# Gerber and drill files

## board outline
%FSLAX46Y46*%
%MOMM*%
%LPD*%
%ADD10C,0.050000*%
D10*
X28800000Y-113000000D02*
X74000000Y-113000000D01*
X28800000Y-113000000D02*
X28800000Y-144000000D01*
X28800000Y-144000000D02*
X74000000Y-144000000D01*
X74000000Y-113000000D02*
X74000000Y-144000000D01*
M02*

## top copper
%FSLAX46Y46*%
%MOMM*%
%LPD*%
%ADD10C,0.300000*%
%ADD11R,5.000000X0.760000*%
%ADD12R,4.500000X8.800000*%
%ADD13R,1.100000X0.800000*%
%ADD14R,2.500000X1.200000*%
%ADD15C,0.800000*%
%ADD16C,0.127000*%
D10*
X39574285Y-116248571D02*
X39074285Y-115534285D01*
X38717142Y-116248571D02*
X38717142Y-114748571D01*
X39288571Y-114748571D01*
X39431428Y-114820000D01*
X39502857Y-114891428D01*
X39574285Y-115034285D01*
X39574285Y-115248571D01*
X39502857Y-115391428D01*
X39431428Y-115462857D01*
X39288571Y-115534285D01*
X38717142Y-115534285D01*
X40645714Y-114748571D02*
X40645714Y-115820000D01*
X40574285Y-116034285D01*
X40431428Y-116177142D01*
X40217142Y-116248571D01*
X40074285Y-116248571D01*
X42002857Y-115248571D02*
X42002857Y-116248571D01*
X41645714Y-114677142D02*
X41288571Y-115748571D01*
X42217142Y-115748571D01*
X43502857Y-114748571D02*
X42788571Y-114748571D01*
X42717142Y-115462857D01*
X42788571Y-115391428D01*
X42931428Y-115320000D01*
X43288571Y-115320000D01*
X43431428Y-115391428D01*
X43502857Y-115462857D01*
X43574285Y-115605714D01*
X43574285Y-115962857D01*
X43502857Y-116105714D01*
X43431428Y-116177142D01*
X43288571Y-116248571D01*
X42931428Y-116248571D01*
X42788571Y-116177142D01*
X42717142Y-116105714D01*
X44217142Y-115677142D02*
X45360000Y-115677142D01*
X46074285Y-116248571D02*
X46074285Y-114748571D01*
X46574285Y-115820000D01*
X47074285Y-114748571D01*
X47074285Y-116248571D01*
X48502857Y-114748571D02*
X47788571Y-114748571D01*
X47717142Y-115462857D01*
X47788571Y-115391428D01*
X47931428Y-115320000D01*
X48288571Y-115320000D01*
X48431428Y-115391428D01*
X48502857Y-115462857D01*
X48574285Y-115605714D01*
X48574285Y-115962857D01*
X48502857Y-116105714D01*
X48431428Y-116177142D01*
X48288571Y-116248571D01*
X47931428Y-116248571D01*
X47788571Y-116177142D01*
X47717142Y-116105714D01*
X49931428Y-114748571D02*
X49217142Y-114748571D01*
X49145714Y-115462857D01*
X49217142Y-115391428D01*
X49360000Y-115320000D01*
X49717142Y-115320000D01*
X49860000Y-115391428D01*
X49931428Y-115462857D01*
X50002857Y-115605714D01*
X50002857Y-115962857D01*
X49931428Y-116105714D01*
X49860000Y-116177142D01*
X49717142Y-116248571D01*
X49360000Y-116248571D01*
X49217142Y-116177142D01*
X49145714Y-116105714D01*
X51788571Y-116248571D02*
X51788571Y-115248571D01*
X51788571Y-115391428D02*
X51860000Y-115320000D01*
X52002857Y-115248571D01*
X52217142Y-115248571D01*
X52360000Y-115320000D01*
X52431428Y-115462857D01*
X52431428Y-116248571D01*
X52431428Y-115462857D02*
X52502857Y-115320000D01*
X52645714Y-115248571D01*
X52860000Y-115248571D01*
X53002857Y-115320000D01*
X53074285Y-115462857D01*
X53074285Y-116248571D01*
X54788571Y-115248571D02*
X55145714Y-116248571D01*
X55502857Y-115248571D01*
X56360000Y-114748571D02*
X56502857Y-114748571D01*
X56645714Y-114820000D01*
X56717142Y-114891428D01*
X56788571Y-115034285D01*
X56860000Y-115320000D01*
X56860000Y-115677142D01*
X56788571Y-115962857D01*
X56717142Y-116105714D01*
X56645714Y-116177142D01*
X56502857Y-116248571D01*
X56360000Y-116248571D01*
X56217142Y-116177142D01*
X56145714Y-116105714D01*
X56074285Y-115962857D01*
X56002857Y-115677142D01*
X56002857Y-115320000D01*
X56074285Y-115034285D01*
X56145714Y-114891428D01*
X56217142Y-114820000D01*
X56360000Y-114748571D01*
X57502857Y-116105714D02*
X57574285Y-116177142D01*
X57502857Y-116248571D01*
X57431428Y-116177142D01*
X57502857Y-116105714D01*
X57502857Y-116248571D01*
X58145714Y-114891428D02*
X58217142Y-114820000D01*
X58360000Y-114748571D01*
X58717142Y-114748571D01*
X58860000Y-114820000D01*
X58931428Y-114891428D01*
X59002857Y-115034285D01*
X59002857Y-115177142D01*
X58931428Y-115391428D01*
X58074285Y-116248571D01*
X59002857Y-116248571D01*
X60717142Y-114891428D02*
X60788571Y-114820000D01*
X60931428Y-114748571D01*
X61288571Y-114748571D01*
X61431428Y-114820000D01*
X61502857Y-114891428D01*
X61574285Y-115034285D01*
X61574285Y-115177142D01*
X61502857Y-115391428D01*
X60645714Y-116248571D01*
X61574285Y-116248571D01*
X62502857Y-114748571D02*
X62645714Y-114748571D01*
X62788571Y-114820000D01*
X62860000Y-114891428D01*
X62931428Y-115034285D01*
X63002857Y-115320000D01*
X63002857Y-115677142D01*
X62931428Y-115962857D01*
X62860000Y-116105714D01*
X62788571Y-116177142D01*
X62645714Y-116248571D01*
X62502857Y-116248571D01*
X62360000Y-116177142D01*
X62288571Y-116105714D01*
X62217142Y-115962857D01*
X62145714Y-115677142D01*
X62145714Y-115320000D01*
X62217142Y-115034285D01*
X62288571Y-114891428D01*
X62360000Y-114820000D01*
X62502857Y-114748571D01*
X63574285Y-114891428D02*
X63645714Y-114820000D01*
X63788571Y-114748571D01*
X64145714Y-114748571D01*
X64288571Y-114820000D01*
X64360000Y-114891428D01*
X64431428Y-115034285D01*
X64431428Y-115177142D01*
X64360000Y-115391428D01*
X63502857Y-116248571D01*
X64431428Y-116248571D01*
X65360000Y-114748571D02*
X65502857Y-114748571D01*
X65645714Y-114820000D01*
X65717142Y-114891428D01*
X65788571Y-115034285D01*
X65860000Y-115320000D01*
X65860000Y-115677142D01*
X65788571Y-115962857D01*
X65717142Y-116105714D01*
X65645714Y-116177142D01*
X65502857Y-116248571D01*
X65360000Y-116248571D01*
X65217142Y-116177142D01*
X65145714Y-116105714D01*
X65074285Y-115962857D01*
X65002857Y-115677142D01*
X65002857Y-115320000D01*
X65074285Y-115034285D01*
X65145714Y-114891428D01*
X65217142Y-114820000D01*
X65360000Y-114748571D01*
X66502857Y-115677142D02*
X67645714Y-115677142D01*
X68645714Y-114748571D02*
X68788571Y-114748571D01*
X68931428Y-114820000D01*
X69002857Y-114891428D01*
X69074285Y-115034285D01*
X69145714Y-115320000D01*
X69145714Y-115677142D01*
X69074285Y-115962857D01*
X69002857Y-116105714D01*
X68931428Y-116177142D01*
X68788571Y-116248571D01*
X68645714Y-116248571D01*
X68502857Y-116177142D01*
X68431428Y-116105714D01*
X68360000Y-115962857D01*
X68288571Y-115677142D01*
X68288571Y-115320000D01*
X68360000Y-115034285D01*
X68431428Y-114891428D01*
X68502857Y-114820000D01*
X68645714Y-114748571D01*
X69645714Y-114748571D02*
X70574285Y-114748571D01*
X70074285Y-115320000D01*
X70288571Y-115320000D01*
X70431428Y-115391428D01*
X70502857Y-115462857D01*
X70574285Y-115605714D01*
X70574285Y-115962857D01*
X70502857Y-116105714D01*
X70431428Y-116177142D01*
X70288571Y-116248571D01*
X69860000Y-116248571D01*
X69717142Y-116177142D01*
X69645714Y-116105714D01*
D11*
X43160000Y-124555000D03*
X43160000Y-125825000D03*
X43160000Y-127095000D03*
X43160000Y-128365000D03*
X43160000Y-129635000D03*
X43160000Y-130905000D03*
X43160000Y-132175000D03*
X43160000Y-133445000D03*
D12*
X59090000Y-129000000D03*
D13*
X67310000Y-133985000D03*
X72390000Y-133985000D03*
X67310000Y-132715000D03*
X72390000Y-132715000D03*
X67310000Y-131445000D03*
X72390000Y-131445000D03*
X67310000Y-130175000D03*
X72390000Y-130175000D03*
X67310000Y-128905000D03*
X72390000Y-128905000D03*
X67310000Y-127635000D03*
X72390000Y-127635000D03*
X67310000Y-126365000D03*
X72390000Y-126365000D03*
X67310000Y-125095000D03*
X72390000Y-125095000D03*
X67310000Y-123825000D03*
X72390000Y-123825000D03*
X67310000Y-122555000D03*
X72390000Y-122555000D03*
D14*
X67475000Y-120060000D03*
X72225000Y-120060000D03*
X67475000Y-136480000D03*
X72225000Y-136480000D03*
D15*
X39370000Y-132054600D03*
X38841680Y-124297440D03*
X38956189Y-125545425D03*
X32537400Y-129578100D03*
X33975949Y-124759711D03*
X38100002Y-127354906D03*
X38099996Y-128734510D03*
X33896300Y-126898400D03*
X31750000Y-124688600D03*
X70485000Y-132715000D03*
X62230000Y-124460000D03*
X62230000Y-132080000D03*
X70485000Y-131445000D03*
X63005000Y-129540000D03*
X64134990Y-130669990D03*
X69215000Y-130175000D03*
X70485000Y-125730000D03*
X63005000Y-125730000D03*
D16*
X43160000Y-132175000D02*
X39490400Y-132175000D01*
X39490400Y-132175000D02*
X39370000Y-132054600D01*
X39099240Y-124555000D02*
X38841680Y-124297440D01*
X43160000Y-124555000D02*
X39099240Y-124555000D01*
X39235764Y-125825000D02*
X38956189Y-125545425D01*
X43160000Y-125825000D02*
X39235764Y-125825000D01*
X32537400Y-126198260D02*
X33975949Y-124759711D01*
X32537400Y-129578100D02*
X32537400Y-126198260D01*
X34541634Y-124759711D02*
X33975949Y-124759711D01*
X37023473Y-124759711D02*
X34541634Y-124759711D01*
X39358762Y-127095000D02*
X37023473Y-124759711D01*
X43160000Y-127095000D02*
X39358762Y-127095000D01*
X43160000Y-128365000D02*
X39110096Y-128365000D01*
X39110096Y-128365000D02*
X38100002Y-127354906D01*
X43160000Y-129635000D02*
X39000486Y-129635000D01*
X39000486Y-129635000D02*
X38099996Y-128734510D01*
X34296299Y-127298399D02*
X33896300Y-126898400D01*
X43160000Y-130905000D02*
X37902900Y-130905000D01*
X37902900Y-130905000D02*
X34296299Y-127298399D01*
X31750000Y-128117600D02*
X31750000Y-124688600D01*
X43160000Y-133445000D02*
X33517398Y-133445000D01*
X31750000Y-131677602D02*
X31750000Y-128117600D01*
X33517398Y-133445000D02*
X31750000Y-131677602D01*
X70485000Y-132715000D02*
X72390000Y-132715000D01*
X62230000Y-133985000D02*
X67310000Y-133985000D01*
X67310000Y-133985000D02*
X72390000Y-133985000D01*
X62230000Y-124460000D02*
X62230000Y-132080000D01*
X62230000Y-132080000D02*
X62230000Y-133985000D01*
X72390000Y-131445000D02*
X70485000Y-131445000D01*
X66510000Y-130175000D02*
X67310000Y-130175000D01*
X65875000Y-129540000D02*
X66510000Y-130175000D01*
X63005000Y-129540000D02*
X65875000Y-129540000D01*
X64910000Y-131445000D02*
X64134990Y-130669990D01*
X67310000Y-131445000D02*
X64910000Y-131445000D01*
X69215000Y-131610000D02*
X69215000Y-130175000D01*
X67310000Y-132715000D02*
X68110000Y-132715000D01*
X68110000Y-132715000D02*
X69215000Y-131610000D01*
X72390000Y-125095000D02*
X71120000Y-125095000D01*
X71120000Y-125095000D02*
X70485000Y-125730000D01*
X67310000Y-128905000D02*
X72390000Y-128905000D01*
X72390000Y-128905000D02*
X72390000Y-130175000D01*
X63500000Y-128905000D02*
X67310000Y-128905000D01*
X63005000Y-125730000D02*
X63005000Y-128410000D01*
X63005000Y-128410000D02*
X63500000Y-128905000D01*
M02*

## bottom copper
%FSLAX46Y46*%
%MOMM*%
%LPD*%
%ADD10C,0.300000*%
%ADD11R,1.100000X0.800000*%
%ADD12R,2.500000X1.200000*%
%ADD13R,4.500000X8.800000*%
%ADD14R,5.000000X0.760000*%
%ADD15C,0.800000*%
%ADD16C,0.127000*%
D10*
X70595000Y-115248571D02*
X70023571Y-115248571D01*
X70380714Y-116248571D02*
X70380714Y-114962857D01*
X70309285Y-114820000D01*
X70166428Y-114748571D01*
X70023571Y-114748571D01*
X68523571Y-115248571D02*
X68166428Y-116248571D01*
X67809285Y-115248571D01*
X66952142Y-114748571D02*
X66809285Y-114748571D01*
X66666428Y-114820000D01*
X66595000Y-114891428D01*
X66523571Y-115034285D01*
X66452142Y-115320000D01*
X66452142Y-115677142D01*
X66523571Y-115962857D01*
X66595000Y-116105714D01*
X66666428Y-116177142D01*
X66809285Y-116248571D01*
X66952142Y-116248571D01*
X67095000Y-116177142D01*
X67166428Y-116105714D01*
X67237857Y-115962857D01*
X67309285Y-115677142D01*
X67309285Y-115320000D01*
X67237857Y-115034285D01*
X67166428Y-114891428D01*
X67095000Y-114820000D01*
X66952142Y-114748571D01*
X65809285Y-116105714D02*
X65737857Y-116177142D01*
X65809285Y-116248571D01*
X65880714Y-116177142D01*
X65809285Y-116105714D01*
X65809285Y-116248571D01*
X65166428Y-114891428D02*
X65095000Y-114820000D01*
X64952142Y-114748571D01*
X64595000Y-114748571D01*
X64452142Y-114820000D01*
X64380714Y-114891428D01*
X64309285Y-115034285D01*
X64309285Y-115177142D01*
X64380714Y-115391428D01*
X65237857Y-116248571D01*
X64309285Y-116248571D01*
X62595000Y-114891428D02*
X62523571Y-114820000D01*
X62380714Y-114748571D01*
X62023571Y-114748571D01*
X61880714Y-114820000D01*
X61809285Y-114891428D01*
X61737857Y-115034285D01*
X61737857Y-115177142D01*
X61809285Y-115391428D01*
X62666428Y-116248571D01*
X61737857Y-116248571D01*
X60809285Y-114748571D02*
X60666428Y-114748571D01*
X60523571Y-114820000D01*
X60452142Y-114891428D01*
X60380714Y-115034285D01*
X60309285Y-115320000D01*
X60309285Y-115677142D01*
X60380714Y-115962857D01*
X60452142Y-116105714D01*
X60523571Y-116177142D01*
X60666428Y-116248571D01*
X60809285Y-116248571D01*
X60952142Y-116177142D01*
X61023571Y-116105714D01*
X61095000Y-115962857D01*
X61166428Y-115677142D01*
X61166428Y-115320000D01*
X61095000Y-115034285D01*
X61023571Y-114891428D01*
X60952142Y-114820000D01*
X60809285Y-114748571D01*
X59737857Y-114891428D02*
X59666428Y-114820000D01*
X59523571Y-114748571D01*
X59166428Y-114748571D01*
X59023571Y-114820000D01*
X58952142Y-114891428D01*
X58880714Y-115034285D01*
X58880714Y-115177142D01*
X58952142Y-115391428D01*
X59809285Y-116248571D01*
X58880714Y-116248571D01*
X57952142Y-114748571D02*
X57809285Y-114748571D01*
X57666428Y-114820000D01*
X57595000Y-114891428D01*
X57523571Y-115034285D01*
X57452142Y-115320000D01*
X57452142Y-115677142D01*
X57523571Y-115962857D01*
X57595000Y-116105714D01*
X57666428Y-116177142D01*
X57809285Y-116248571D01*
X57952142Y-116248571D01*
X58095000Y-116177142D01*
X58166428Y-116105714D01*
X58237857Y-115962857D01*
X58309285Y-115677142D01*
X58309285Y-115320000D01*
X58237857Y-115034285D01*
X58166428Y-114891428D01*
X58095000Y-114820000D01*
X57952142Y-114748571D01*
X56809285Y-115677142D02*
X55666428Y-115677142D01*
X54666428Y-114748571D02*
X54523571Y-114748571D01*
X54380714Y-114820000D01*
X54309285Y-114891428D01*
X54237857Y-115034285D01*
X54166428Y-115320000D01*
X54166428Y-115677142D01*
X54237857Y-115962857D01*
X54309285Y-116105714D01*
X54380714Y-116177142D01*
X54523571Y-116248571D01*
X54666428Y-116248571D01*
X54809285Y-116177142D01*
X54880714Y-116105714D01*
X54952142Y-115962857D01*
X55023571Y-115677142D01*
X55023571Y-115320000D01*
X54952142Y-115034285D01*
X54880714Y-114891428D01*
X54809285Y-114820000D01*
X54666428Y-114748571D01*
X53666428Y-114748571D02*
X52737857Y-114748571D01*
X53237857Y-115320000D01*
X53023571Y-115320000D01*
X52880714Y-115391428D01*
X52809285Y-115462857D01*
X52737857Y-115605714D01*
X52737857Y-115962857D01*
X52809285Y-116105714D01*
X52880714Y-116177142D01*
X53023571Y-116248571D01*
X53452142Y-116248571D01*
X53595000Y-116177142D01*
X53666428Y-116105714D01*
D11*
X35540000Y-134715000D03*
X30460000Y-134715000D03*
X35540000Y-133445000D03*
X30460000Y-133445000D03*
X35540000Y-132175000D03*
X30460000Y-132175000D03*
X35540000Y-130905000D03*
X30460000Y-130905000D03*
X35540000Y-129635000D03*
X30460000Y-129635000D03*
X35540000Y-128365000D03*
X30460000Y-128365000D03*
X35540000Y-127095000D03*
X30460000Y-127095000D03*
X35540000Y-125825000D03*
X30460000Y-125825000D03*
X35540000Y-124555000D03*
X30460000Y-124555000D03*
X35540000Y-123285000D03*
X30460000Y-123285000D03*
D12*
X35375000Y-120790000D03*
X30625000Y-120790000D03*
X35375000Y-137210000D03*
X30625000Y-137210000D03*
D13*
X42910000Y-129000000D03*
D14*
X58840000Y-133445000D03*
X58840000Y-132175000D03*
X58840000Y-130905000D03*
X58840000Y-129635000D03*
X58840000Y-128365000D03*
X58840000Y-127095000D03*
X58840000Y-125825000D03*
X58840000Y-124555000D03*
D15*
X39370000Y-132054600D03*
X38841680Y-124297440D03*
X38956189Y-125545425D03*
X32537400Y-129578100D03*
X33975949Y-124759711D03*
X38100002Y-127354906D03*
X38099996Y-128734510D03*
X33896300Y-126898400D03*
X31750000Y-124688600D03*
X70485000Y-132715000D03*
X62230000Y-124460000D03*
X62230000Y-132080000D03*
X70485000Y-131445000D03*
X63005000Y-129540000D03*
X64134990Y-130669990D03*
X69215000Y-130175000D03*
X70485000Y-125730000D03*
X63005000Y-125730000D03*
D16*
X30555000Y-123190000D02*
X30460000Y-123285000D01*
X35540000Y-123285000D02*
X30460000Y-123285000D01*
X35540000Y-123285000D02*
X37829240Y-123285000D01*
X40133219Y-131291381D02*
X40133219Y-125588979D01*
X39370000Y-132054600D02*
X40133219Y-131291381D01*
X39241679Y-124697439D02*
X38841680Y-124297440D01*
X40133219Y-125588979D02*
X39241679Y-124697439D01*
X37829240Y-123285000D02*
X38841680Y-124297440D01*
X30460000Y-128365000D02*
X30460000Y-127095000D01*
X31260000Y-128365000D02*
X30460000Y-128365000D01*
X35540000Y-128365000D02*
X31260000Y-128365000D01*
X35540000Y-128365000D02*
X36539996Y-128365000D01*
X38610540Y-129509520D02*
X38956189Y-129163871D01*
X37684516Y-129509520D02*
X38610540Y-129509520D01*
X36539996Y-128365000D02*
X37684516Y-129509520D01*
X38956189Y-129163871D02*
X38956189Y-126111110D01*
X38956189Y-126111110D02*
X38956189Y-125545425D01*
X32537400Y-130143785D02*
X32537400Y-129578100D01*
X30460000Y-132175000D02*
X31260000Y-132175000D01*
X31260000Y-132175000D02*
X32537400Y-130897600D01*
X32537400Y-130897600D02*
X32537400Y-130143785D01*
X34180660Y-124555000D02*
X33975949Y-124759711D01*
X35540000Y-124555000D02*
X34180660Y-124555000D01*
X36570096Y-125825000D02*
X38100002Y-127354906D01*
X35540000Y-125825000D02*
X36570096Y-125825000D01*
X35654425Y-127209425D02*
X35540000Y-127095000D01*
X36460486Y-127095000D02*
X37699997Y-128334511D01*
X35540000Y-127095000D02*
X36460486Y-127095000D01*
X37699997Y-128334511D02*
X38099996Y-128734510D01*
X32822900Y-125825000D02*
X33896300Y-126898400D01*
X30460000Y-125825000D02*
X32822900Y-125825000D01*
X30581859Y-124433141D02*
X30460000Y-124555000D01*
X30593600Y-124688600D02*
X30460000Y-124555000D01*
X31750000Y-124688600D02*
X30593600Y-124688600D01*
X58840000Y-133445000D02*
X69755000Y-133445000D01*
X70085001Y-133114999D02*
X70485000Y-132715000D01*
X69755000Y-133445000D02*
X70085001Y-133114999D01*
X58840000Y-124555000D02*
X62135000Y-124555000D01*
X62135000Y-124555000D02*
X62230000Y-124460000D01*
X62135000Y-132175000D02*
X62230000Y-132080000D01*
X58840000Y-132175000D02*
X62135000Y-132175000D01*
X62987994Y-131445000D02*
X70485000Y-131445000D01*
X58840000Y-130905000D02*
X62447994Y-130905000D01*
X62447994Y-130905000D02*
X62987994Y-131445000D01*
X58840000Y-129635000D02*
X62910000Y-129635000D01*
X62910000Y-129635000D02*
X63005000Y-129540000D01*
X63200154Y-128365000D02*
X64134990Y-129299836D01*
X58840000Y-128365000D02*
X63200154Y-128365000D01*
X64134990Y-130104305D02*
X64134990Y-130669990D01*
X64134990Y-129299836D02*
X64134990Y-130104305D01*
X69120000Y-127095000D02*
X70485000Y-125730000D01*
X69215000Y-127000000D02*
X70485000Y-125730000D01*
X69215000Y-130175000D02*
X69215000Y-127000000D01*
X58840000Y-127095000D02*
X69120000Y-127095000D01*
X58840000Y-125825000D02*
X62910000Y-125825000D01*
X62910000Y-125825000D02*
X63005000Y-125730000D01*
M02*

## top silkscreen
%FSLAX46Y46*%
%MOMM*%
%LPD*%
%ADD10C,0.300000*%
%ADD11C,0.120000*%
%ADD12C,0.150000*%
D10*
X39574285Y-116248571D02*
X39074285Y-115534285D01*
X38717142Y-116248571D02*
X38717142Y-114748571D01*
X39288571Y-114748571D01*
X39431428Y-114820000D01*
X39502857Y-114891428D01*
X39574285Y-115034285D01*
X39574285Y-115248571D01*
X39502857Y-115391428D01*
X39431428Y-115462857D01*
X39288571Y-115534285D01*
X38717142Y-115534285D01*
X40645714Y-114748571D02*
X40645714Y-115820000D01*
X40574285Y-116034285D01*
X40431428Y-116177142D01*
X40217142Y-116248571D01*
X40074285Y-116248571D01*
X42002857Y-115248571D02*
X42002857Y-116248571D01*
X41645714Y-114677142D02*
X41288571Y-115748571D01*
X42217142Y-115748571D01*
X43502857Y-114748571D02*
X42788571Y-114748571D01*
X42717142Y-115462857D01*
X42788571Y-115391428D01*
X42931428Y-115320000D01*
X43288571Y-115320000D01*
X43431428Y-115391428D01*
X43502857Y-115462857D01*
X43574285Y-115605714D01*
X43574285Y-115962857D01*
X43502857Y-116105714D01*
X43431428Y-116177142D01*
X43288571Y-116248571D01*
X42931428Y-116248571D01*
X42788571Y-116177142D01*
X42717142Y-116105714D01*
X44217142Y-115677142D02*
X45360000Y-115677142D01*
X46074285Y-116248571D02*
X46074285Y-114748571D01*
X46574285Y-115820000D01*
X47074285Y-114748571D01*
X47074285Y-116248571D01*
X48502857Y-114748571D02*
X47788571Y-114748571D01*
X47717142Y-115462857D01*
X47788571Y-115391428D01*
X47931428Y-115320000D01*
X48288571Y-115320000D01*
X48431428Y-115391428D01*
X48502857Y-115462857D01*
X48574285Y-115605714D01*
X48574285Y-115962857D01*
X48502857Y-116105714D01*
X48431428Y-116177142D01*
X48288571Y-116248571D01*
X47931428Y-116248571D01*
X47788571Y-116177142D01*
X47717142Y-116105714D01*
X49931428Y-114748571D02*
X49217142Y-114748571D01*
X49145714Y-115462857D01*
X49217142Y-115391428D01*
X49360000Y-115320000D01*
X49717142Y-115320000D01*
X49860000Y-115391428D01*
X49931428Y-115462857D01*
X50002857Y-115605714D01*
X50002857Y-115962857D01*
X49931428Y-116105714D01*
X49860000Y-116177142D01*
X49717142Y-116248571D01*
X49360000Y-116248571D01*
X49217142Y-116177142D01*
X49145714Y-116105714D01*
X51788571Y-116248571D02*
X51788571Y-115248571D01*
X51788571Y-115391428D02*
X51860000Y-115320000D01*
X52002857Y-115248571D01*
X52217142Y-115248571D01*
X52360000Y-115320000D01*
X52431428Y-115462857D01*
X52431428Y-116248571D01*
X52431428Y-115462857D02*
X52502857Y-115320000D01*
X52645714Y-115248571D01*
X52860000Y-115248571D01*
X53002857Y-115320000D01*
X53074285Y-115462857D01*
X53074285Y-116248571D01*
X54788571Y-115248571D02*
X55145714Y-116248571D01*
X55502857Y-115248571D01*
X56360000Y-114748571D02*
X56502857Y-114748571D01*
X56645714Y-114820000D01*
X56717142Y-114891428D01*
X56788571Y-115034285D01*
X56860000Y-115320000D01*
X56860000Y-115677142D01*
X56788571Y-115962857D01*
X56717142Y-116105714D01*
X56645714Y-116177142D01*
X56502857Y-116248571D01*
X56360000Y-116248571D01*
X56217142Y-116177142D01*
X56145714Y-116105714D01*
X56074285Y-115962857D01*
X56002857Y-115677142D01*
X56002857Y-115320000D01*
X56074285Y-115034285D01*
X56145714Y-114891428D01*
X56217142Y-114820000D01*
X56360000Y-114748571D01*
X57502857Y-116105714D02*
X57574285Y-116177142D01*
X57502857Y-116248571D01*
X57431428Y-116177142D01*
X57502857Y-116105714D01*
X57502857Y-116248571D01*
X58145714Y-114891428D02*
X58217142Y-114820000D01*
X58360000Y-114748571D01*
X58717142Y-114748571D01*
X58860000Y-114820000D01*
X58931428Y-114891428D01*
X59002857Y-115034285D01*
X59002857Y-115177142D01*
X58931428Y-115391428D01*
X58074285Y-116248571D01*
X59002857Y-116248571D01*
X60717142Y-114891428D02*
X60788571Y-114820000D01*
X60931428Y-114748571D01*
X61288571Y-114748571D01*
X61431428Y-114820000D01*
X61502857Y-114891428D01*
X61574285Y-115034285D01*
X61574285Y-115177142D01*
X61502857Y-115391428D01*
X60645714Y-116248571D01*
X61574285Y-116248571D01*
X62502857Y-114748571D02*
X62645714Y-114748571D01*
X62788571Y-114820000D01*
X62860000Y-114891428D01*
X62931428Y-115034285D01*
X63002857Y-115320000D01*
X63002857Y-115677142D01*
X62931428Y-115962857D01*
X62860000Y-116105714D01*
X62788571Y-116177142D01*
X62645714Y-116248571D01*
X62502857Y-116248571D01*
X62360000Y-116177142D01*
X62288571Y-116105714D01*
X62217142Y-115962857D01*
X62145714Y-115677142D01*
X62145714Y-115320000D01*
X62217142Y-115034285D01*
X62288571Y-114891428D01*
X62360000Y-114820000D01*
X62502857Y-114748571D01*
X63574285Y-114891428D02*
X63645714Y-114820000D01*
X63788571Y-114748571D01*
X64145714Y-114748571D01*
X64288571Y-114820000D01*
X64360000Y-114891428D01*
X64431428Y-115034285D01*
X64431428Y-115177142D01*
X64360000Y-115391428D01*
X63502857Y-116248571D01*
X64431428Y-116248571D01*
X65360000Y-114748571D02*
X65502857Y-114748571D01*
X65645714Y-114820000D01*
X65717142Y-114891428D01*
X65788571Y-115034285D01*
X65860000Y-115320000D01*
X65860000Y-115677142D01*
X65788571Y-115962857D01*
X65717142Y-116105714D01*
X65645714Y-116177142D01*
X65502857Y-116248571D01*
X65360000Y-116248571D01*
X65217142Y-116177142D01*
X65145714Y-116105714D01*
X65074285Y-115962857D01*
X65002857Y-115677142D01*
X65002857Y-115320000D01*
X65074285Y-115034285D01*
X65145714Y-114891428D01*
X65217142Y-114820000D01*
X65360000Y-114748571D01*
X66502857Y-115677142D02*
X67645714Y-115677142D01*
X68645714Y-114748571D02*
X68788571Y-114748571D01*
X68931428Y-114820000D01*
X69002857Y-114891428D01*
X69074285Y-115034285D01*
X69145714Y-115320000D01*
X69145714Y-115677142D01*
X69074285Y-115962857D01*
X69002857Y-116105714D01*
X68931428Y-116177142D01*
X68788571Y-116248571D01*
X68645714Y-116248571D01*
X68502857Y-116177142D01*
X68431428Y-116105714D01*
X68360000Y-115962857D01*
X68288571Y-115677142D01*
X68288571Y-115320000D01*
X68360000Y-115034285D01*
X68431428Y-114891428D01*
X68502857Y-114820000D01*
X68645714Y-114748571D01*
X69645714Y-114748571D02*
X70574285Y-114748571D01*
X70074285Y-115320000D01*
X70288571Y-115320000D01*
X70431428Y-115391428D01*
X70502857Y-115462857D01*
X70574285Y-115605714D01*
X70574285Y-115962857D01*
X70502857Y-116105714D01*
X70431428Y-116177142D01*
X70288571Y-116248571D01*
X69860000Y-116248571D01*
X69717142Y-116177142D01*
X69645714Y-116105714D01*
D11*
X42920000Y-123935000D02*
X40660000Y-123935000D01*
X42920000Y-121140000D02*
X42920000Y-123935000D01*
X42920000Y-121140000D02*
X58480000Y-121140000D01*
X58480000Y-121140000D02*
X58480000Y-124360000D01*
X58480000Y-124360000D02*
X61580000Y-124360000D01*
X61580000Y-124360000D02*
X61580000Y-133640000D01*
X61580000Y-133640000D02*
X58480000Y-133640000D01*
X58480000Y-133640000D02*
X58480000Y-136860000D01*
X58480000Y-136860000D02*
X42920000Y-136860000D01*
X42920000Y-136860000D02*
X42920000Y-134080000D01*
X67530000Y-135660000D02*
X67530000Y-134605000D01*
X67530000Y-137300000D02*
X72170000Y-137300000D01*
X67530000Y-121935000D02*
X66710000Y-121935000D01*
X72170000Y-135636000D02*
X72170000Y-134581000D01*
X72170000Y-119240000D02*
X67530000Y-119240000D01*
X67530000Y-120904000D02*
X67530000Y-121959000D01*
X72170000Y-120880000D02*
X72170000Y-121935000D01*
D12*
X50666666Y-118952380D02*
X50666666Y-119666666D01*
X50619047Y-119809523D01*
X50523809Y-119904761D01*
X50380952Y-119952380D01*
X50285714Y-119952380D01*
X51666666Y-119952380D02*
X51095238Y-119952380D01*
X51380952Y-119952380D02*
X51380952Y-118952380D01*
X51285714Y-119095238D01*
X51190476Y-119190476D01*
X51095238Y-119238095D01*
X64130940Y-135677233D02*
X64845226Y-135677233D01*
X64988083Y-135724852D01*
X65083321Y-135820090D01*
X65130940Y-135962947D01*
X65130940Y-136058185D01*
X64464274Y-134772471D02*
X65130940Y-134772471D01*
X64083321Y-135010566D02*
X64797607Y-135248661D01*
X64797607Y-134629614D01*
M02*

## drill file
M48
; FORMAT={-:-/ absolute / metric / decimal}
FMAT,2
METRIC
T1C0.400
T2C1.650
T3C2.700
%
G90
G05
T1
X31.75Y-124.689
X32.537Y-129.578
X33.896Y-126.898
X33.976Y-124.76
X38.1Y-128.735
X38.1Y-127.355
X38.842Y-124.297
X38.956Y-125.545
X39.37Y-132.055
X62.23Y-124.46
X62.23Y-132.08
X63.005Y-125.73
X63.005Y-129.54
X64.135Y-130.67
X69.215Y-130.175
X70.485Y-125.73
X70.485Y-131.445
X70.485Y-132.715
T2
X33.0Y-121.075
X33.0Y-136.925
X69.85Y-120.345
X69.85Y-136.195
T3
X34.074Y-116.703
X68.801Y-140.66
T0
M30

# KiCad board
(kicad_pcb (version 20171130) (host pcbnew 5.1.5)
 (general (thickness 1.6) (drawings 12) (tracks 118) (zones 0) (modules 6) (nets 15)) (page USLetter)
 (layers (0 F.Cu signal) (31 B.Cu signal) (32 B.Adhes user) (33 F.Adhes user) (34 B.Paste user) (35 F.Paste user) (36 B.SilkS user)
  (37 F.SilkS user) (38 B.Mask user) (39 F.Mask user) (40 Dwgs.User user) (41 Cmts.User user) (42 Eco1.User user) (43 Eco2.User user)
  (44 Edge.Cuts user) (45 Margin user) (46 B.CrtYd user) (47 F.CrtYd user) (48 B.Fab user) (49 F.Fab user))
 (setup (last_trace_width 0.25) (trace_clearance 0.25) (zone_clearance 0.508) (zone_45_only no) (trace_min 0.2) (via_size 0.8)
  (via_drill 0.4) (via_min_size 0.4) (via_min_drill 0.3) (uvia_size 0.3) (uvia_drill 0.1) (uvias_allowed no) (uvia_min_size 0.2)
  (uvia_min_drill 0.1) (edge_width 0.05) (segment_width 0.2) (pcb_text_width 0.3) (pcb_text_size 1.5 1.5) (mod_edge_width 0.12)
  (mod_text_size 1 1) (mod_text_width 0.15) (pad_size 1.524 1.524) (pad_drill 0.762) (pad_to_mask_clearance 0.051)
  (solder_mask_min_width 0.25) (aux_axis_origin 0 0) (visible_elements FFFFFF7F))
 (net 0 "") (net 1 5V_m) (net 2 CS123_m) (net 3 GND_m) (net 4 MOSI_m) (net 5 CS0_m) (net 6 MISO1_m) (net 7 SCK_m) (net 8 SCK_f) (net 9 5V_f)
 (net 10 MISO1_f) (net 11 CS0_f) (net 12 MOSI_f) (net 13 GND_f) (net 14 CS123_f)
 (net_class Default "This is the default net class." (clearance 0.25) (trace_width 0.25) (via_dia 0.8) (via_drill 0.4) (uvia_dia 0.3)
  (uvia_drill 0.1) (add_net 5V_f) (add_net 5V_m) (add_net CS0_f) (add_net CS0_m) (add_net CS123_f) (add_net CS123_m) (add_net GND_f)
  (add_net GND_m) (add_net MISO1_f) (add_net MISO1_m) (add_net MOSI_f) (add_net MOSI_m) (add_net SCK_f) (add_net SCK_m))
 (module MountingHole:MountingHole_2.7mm (layer F.Cu) (at 68.80098 140.66012)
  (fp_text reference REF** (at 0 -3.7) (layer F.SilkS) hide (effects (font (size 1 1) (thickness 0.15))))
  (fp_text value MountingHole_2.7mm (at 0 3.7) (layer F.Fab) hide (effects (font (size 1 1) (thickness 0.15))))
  (pad 1 np_thru_hole circle (at 0 0) (size 2.7 2.7) (drill 2.7) (layers *.Cu *.Mask)))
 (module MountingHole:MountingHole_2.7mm (layer F.Cu) (at 34.0741 116.70284)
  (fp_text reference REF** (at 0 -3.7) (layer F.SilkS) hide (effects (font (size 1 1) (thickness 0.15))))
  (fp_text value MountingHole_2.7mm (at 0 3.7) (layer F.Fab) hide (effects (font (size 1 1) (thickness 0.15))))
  (pad 1 np_thru_hole circle (at 0 0) (size 2.7 2.7) (drill 2.7) (layers *.Cu *.Mask)))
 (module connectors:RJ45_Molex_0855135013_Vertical (layer F.Cu) (at 51 129)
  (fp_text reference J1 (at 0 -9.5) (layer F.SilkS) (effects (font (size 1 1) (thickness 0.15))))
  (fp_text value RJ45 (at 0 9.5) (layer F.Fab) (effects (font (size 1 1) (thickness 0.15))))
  (fp_line (start -8.08 -5.065) (end -10.34 -5.065) (layer F.SilkS) (width 0.12))
  (fp_line (start -8.08 -7.86) (end -8.08 -5.065) (layer F.SilkS) (width 0.12))
  (fp_line (start -8.08 -7.86) (end 7.48 -7.86) (layer F.SilkS) (width 0.12))
  (fp_line (start 7.48 -7.86) (end 7.48 -4.64) (layer F.SilkS) (width 0.12))
  (fp_line (start 7.48 -4.64) (end 10.58 -4.64) (layer F.SilkS) (width 0.12))
  (fp_line (start 10.58 -4.64) (end 10.58 4.64) (layer F.SilkS) (width 0.12))
  (fp_line (start 10.58 4.64) (end 7.48 4.64) (layer F.SilkS) (width 0.12))
  (fp_line (start 7.48 4.64) (end 7.48 7.86) (layer F.SilkS) (width 0.12))
  (fp_line (start 7.48 7.86) (end -8.08 7.86) (layer F.SilkS) (width 0.12))
  (fp_line (start -8.08 7.86) (end -8.08 5.08) (layer F.SilkS) (width 0.12))
  (pad 1 smd rect (at -7.84 -4.445 270) (size 0.76 5) (layers F.Cu F.Paste F.Mask) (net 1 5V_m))
  (pad 2 smd rect (at -7.84 -3.175 270) (size 0.76 5) (layers F.Cu F.Paste F.Mask) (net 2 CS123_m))
  (pad 3 smd rect (at -7.84 -1.905 270) (size 0.76 5) (layers F.Cu F.Paste F.Mask) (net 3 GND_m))
  (pad 4 smd rect (at -7.84 -0.635 270) (size 0.76 5) (layers F.Cu F.Paste F.Mask) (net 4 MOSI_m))
  (pad 5 smd rect (at -7.84 0.635 270) (size 0.76 5) (layers F.Cu F.Paste F.Mask) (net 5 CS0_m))
  (pad 6 smd rect (at -7.84 1.905 270) (size 0.76 5) (layers F.Cu F.Paste F.Mask) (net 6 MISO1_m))
  (pad 7 smd rect (at -7.84 3.175 270) (size 0.76 5) (layers F.Cu F.Paste F.Mask) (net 1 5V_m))
  (pad 8 smd rect (at -7.84 4.445 270) (size 0.76 5) (layers F.Cu F.Paste F.Mask) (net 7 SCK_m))
  (pad L smd rect (at 8.09 0 270) (size 8.8 4.5) (layers F.Cu F.Paste F.Mask)))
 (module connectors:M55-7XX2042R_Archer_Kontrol (layer B.Cu) (at 33 129 90)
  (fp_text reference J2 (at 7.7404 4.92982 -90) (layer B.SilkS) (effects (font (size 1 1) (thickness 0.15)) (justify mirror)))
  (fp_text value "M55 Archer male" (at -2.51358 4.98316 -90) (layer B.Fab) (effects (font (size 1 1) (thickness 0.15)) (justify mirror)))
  (pad 1 smd rect (at -5.715 2.54 90) (size 0.8 1.1) (layers B.Cu B.Paste B.Mask))
  (pad 2 smd rect (at -5.715 -2.54 90) (size 0.8 1.1) (layers B.Cu B.Paste B.Mask))
  (pad 3 smd rect (at -4.445 2.54 90) (size 0.8 1.1) (layers B.Cu B.Paste B.Mask))
  (pad 4 smd rect (at -4.445 -2.54 90) (size 0.8 1.1) (layers B.Cu B.Paste B.Mask))
  (pad 5 smd rect (at -3.175 2.54 90) (size 0.8 1.1) (layers B.Cu B.Paste B.Mask))
  (pad 6 smd rect (at -3.175 -2.54 90) (size 0.8 1.1) (layers B.Cu B.Paste B.Mask) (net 3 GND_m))
  (pad 7 smd rect (at -1.905 2.54 90) (size 0.8 1.1) (layers B.Cu B.Paste B.Mask))
  (pad 8 smd rect (at -1.905 -2.54 90) (size 0.8 1.1) (layers B.Cu B.Paste B.Mask))
  (pad 9 smd rect (at -0.635 2.54 90) (size 0.8 1.1) (layers B.Cu B.Paste B.Mask))
  (pad 10 smd rect (at -0.635 -2.54 90) (size 0.8 1.1) (layers B.Cu B.Paste B.Mask))
  (pad 11 smd rect (at 0.635 2.54 90) (size 0.8 1.1) (layers B.Cu B.Paste B.Mask) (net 2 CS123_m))
  (pad 12 smd rect (at 0.635 -2.54 90) (size 0.8 1.1) (layers B.Cu B.Paste B.Mask) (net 2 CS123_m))
  (pad 13 smd rect (at 1.905 2.54 90) (size 0.8 1.1) (layers B.Cu B.Paste B.Mask) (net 5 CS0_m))
  (pad 14 smd rect (at 1.905 -2.54 90) (size 0.8 1.1) (layers B.Cu B.Paste B.Mask) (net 2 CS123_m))
  (pad 15 smd rect (at 3.175 2.54 90) (size 0.8 1.1) (layers B.Cu B.Paste B.Mask) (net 4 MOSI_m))
  (pad 16 smd rect (at 3.175 -2.54 90) (size 0.8 1.1) (layers B.Cu B.Paste B.Mask) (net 6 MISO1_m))
  (pad 17 smd rect (at 4.445 2.54 90) (size 0.8 1.1) (layers B.Cu B.Paste B.Mask) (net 3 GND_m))
  (pad 18 smd rect (at 4.445 -2.54 90) (size 0.8 1.1) (layers B.Cu B.Paste B.Mask) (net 7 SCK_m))
  (pad 19 smd rect (at 5.715 2.54 90) (size 0.8 1.1) (layers B.Cu B.Paste B.Mask) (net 1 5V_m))
  (pad 20 smd rect (at 5.715 -2.54 90) (size 0.8 1.1) (layers B.Cu B.Paste B.Mask) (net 1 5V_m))
  (pad "" np_thru_hole circle (at 7.925 0 90) (size 1.65 1.65) (drill 1.65) (layers *.Cu *.Mask))
  (pad "" np_thru_hole circle (at -7.925 0 90) (size 1.65 1.65) (drill 1.65) (layers *.Cu *.Mask))
  (pad "" smd rect (at 8.21 2.375 90) (size 1.2 2.5) (layers B.Cu B.Paste B.Mask))
  (pad "" smd rect (at 8.21 -2.375 90) (size 1.2 2.5) (layers B.Cu B.Paste B.Mask))
  (pad "" smd rect (at -8.21 2.375 90) (size 1.2 2.5) (layers B.Cu B.Paste B.Mask))
  (pad "" smd rect (at -8.21 -2.375 90) (size 1.2 2.5) (layers B.Cu B.Paste B.Mask)))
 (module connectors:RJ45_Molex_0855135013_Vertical (layer B.Cu) (at 51 129 180)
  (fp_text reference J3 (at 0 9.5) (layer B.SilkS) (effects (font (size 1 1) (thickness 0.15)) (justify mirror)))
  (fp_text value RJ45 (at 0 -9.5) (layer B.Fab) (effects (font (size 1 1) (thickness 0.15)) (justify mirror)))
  (pad L smd rect (at 8.09 0 270) (size 8.8 4.5) (layers B.Cu B.Paste B.Mask))
  (pad 8 smd rect (at -7.84 -4.445 270) (size 0.76 5) (layers B.Cu B.Paste B.Mask) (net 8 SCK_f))
  (pad 7 smd rect (at -7.84 -3.175 270) (size 0.76 5) (layers B.Cu B.Paste B.Mask) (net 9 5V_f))
  (pad 6 smd rect (at -7.84 -1.905 270) (size 0.76 5) (layers B.Cu B.Paste B.Mask) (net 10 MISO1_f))
  (pad 5 smd rect (at -7.84 -0.635 270) (size 0.76 5) (layers B.Cu B.Paste B.Mask) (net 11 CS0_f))
  (pad 4 smd rect (at -7.84 0.635 270) (size 0.76 5) (layers B.Cu B.Paste B.Mask) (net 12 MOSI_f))
  (pad 3 smd rect (at -7.84 1.905 270) (size 0.76 5) (layers B.Cu B.Paste B.Mask) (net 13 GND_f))
  (pad 2 smd rect (at -7.84 3.175 270) (size 0.76 5) (layers B.Cu B.Paste B.Mask) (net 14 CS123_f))
  (pad 1 smd rect (at -7.84 4.445 270) (size 0.76 5) (layers B.Cu B.Paste B.Mask) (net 9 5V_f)))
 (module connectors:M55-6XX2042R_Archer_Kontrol (layer F.Cu) (at 69.85 128.27 90)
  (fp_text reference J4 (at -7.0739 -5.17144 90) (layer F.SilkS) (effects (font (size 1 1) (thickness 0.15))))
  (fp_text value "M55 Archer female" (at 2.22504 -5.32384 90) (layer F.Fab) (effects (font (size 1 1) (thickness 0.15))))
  (fp_line (start -7.39 -2.32) (end -6.335 -2.32) (layer F.SilkS) (width 0.12))
  (fp_line (start -9.03 -2.32) (end -9.03 2.32) (layer F.SilkS) (width 0.12))
  (fp_line (start 6.335 -2.32) (end 6.335 -3.14) (layer F.SilkS) (width 0.12))
  (fp_line (start -7.366 2.32) (end -6.311 2.32) (layer F.SilkS) (width 0.12))
  (fp_line (start 9.03 2.32) (end 9.03 -2.32) (layer F.SilkS) (width 0.12))
  (fp_line (start 7.366 -2.32) (end 6.311 -2.32) (layer F.SilkS) (width 0.12))
  (fp_line (start 7.39 2.32) (end 6.335 2.32) (layer F.SilkS) (width 0.12))
  (pad 19 smd rect (at -5.715 -2.54 90) (size 0.8 1.1) (layers F.Cu F.Paste F.Mask) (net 9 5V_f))
  (pad 20 smd rect (at -5.715 2.54 90) (size 0.8 1.1) (layers F.Cu F.Paste F.Mask) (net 9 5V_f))
  (pad 17 smd rect (at -4.445 -2.54 90) (size 0.8 1.1) (layers F.Cu F.Paste F.Mask) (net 13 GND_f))
  (pad 18 smd rect (at -4.445 2.54 90) (size 0.8 1.1) (layers F.Cu F.Paste F.Mask) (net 8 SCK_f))
  (pad 15 smd rect (at -3.175 -2.54 90) (size 0.8 1.1) (layers F.Cu F.Paste F.Mask) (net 12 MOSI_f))
  (pad 16 smd rect (at -3.175 2.54 90) (size 0.8 1.1) (layers F.Cu F.Paste F.Mask) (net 10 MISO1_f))
  (pad 13 smd rect (at -1.905 -2.54 90) (size 0.8 1.1) (layers F.Cu F.Paste F.Mask) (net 11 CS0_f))
  (pad 14 smd rect (at -1.905 2.54 90) (size 0.8 1.1) (layers F.Cu F.Paste F.Mask) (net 14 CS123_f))
  (pad 11 smd rect (at -0.635 -2.54 90) (size 0.8 1.1) (layers F.Cu F.Paste F.Mask) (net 14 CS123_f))
  (pad 12 smd rect (at -0.635 2.54 90) (size 0.8 1.1) (layers F.Cu F.Paste F.Mask) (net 14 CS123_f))
  (pad 9 smd rect (at 0.635 -2.54 90) (size 0.8 1.1) (layers F.Cu F.Paste F.Mask))
  (pad 10 smd rect (at 0.635 2.54 90) (size 0.8 1.1) (layers F.Cu F.Paste F.Mask))
  (pad 7 smd rect (at 1.905 -2.54 90) (size 0.8 1.1) (layers F.Cu F.Paste F.Mask))
  (pad 8 smd rect (at 1.905 2.54 90) (size 0.8 1.1) (layers F.Cu F.Paste F.Mask))
  (pad 5 smd rect (at 3.175 -2.54 90) (size 0.8 1.1) (layers F.Cu F.Paste F.Mask))
  (pad 6 smd rect (at 3.175 2.54 90) (size 0.8 1.1) (layers F.Cu F.Paste F.Mask) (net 13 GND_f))
  (pad 3 smd rect (at 4.445 -2.54 90) (size 0.8 1.1) (layers F.Cu F.Paste F.Mask))
  (pad 4 smd rect (at 4.445 2.54 90) (size 0.8 1.1) (layers F.Cu F.Paste F.Mask))
  (pad 1 smd rect (at 5.715 -2.54 90) (size 0.8 1.1) (layers F.Cu F.Paste F.Mask))
  (pad 2 smd rect (at 5.715 2.54 90) (size 0.8 1.1) (layers F.Cu F.Paste F.Mask))
  (pad "" np_thru_hole circle (at 7.925 0 90) (size 1.65 1.65) (drill 1.65) (layers *.Cu *.Mask))
  (pad "" np_thru_hole circle (at -7.925 0 90) (size 1.65 1.65) (drill 1.65) (layers *.Cu *.Mask))
  (pad "" smd rect (at 8.21 -2.375 90) (size 1.2 2.5) (layers F.Cu F.Paste F.Mask))
  (pad "" smd rect (at 8.21 2.375 90) (size 1.2 2.5) (layers F.Cu F.Paste F.Mask))
  (pad "" smd rect (at -8.21 -2.375 90) (size 1.2 2.5) (layers F.Cu F.Paste F.Mask))
  (pad "" smd rect (at -8.21 2.375 90) (size 1.2 2.5) (layers F.Cu F.Paste F.Mask)))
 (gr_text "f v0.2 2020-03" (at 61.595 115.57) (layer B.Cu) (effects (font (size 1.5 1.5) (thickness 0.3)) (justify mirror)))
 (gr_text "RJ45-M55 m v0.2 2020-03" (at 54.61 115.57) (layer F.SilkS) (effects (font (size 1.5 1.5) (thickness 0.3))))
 (gr_line (start 28.8 113) (end 74 113) (layer Edge.Cuts) (width 0.05))
 (gr_line (start 28.8 113) (end 28.8 144) (layer Edge.Cuts) (width 0.05))
 (gr_line (start 28.8 144) (end 74 144) (layer Edge.Cuts) (width 0.05))
 (gr_line (start 74 113) (end 74 144) (layer Edge.Cuts) (width 0.05))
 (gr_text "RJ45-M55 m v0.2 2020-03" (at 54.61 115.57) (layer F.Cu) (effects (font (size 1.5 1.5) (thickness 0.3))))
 (segment (start 30.555 123.19) (end 30.46 123.285) (width 0.127) (layer B.Cu) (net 1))
 (segment (start 35.54 123.285) (end 30.46 123.285) (width 0.127) (layer B.Cu) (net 1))
 (segment (start 43.16 132.175) (end 39.4904 132.175) (width 0.127) (layer F.Cu) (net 1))
 (segment (start 39.4904 132.175) (end 39.37 132.0546) (width 0.127) (layer F.Cu) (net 1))
 (via (at 39.37 132.0546) (size 0.8) (drill 0.4) (layers F.Cu B.Cu) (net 1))
 (segment (start 35.54 123.285) (end 37.82924 123.285) (width 0.127) (layer B.Cu) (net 1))
 (segment (start 39.09924 124.555) (end 38.84168 124.29744) (width 0.127) (layer F.Cu) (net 1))
 (segment (start 40.133219 131.291381) (end 40.133219 125.588979) (width 0.127) (layer B.Cu) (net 1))
 (segment (start 39.37 132.0546) (end 40.133219 131.291381) (width 0.127) (layer B.Cu) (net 1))
 (via (at 38.84168 124.29744) (size 0.8) (drill 0.4) (layers F.Cu B.Cu) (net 1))
 (segment (start 39.241679 124.697439) (end 38.84168 124.29744) (width 0.127) (layer B.Cu) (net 1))
 (segment (start 43.16 124.555) (end 39.09924 124.555) (width 0.127) (layer F.Cu) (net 1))
 (segment (start 40.133219 125.588979) (end 39.241679 124.697439) (width 0.127) (layer B.Cu) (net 1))
 (segment (start 37.82924 123.285) (end 38.84168 124.29744) (width 0.127) (layer B.Cu) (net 1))
 (segment (start 30.46 128.365) (end 30.46 127.095) (width 0.127) (layer B.Cu) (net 2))
 (segment (start 31.26 128.365) (end 30.46 128.365) (width 0.127) (layer B.Cu) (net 2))
 (segment (start 35.54 128.365) (end 31.26 128.365) (width 0.127) (layer B.Cu) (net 2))
 (segment (start 35.54 128.365) (end 36.539996 128.365) (width 0.127) (layer B.Cu) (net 2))
 (segment (start 39.235764 125.825) (end 38.956189 125.545425) (width 0.127) (layer F.Cu) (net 2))
 (segment (start 38.61054 129.50952) (end 38.956189 129.163871) (width 0.127) (layer B.Cu) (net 2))
 (segment (start 37.684516 129.50952) (end 38.61054 129.50952) (width 0.127) (layer B.Cu) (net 2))
 (via (at 38.956189 125.545425) (size 0.8) (drill 0.4) (layers F.Cu B.Cu) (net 2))
 (segment (start 43.16 125.825) (end 39.235764 125.825) (width 0.127) (layer F.Cu) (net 2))
 (segment (start 36.539996 128.365) (end 37.684516 129.50952) (width 0.127) (layer B.Cu) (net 2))
 (segment (start 38.956189 129.163871) (end 38.956189 126.11111) (width 0.127) (layer B.Cu) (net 2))
 (segment (start 38.956189 126.11111) (end 38.956189 125.545425) (width 0.127) (layer B.Cu) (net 2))
 (via (at 32.5374 129.5781) (size 0.8) (drill 0.4) (layers F.Cu B.Cu) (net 3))
 (segment (start 32.5374 130.143785) (end 32.5374 129.5781) (width 0.127) (layer B.Cu) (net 3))
 (segment (start 30.46 132.175) (end 31.26 132.175) (width 0.127) (layer B.Cu) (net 3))
 (segment (start 31.26 132.175) (end 32.5374 130.8976) (width 0.127) (layer B.Cu) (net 3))
 (segment (start 32.5374 130.8976) (end 32.5374 130.143785) (width 0.127) (layer B.Cu) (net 3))
 (segment (start 34.18066 124.555) (end 33.975949 124.759711) (width 0.127) (layer B.Cu) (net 3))
 (via (at 33.975949 124.759711) (size 0.8) (drill 0.4) (layers F.Cu B.Cu) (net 3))
 (segment (start 35.54 124.555) (end 34.18066 124.555) (width 0.127) (layer B.Cu) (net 3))
 (segment (start 32.5374 126.19826) (end 33.975949 124.759711) (width 0.127) (layer F.Cu) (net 3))
 (segment (start 32.5374 129.5781) (end 32.5374 126.19826) (width 0.127) (layer F.Cu) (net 3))
 (segment (start 34.541634 124.759711) (end 33.975949 124.759711) (width 0.127) (layer F.Cu) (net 3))
 (segment (start 37.023473 124.759711) (end 34.541634 124.759711) (width 0.127) (layer F.Cu) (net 3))
 (segment (start 39.358762 127.095) (end 37.023473 124.759711) (width 0.127) (layer F.Cu) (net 3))
 (segment (start 43.16 127.095) (end 39.358762 127.095) (width 0.127) (layer F.Cu) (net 3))
 (segment (start 43.16 128.365) (end 39.110096 128.365) (width 0.127) (layer F.Cu) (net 4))
 (segment (start 36.570096 125.825) (end 38.100002 127.354906) (width 0.127) (layer B.Cu) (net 4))
 (segment (start 35.54 125.825) (end 36.570096 125.825) (width 0.127) (layer B.Cu) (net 4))
 (segment (start 39.110096 128.365) (end 38.100002 127.354906) (width 0.127) (layer F.Cu) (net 4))
 (via (at 38.100002 127.354906) (size 0.8) (drill 0.4) (layers F.Cu B.Cu) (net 4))
 (segment (start 35.654425 127.209425) (end 35.54 127.095) (width 0.127) (layer B.Cu) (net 5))
 (via (at 38.099996 128.73451) (size 0.8) (drill 0.4) (layers F.Cu B.Cu) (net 5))
 (segment (start 36.460486 127.095) (end 37.699997 128.334511) (width 0.127) (layer B.Cu) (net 5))
 (segment (start 43.16 129.635) (end 39.000486 129.635) (width 0.127) (layer F.Cu) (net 5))
 (segment (start 35.54 127.095) (end 36.460486 127.095) (width 0.127) (layer B.Cu) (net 5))
 (segment (start 37.699997 128.334511) (end 38.099996 128.73451) (width 0.127) (layer B.Cu) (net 5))
 (segment (start 39.000486 129.635) (end 38.099996 128.73451) (width 0.127) (layer F.Cu) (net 5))
 (segment (start 34.296299 127.298399) (end 33.8963 126.8984) (width 0.127) (layer F.Cu) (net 6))
 (segment (start 43.16 130.905) (end 37.9029 130.905) (width 0.127) (layer F.Cu) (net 6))
 (segment (start 37.9029 130.905) (end 34.296299 127.298399) (width 0.127) (layer F.Cu) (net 6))
 (via (at 33.8963 126.8984) (size 0.8) (drill 0.4) (layers F.Cu B.Cu) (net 6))
 (segment (start 32.8229 125.825) (end 33.8963 126.8984) (width 0.127) (layer B.Cu) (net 6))
 (segment (start 30.46 125.825) (end 32.8229 125.825) (width 0.127) (layer B.Cu) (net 6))
 (segment (start 30.581859 124.433141) (end 30.46 124.555) (width 0.127) (layer B.Cu) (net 7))
 (via (at 31.75 124.6886) (size 0.8) (drill 0.4) (layers F.Cu B.Cu) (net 7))
 (segment (start 30.5936 124.6886) (end 30.46 124.555) (width 0.127) (layer B.Cu) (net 7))
 (segment (start 31.75 124.6886) (end 30.5936 124.6886) (width 0.127) (layer B.Cu) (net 7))
 (segment (start 31.75 128.1176) (end 31.75 124.6886) (width 0.127) (layer F.Cu) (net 7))
 (segment (start 43.16 133.445) (end 33.517398 133.445) (width 0.127) (layer F.Cu) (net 7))
 (segment (start 31.75 131.677602) (end 31.75 128.1176) (width 0.127) (layer F.Cu) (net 7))
 (segment (start 33.517398 133.445) (end 31.75 131.677602) (width 0.127) (layer F.Cu) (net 7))
 (via (at 70.485 132.715) (size 0.8) (drill 0.4) (layers F.Cu B.Cu) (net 8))
 (segment (start 70.485 132.715) (end 72.39 132.715) (width 0.127) (layer F.Cu) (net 8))
 (segment (start 58.84 133.445) (end 69.755 133.445) (width 0.127) (layer B.Cu) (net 8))
 (segment (start 70.085001 133.114999) (end 70.485 132.715) (width 0.127) (layer B.Cu) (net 8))
 (segment (start 69.755 133.445) (end 70.085001 133.114999) (width 0.127) (layer B.Cu) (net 8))
 (via (at 62.23 124.46) (size 0.8) (drill 0.4) (layers F.Cu B.Cu) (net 9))
 (segment (start 58.84 124.555) (end 62.135 124.555) (width 0.127) (layer B.Cu) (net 9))
 (segment (start 62.135 124.555) (end 62.23 124.46) (width 0.127) (layer B.Cu) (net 9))
 (segment (start 62.23 133.985) (end 67.31 133.985) (width 0.127) (layer F.Cu) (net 9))
 (segment (start 67.31 133.985) (end 72.39 133.985) (width 0.127) (layer F.Cu) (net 9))
 (via (at 62.23 132.08) (size 0.8) (drill 0.4) (layers F.Cu B.Cu) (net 9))
 (segment (start 62.135 132.175) (end 62.23 132.08) (width 0.127) (layer B.Cu) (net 9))
 (segment (start 58.84 132.175) (end 62.135 132.175) (width 0.127) (layer B.Cu) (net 9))
 (segment (start 62.23 124.46) (end 62.23 132.08) (width 0.127) (layer F.Cu) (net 9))
 (segment (start 62.23 132.08) (end 62.23 133.985) (width 0.127) (layer F.Cu) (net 9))
 (segment (start 72.39 131.445) (end 70.485 131.445) (width 0.127) (layer F.Cu) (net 10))
 (via (at 70.485 131.445) (size 0.8) (drill 0.4) (layers F.Cu B.Cu) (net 10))
 (segment (start 62.987994 131.445) (end 70.485 131.445) (width 0.127) (layer B.Cu) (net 10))
 (segment (start 58.84 130.905) (end 62.447994 130.905) (width 0.127) (layer B.Cu) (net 10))
 (segment (start 62.447994 130.905) (end 62.987994 131.445) (width 0.127) (layer B.Cu) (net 10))
 (segment (start 58.84 129.635) (end 62.91 129.635) (width 0.127) (layer B.Cu) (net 11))
 (via (at 63.005 129.54) (size 0.8) (drill 0.4) (layers F.Cu B.Cu) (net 11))
 (segment (start 62.91 129.635) (end 63.005 129.54) (width 0.127) (layer B.Cu) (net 11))
 (segment (start 66.51 130.175) (end 67.31 130.175) (width 0.127) (layer F.Cu) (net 11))
 (segment (start 65.875 129.54) (end 66.51 130.175) (width 0.127) (layer F.Cu) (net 11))
 (segment (start 63.005 129.54) (end 65.875 129.54) (width 0.127) (layer F.Cu) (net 11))
 (segment (start 64.91 131.445) (end 64.13499 130.66999) (width 0.127) (layer F.Cu) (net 12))
 (segment (start 67.31 131.445) (end 64.91 131.445) (width 0.127) (layer F.Cu) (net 12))
 (via (at 64.13499 130.66999) (size 0.8) (drill 0.4) (layers F.Cu B.Cu) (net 12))
 (segment (start 63.200154 128.365) (end 64.13499 129.299836) (width 0.127) (layer B.Cu) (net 12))
 (segment (start 58.84 128.365) (end 63.200154 128.365) (width 0.127) (layer B.Cu) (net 12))
 (segment (start 64.13499 130.104305) (end 64.13499 130.66999) (width 0.127) (layer B.Cu) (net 12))
 (segment (start 64.13499 129.299836) (end 64.13499 130.104305) (width 0.127) (layer B.Cu) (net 12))
 (via (at 69.215 130.175) (size 0.8) (drill 0.4) (layers F.Cu B.Cu) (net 13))
 (segment (start 69.215 131.61) (end 69.215 130.175) (width 0.127) (layer F.Cu) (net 13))
 (segment (start 67.31 132.715) (end 68.11 132.715) (width 0.127) (layer F.Cu) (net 13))
 (segment (start 68.11 132.715) (end 69.215 131.61) (width 0.127) (layer F.Cu) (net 13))
 (segment (start 72.39 125.095) (end 71.12 125.095) (width 0.127) (layer F.Cu) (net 13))
 (segment (start 69.12 127.095) (end 70.485 125.73) (width 0.127) (layer B.Cu) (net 13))
 (via (at 70.485 125.73) (size 0.8) (drill 0.4) (layers F.Cu B.Cu) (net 13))
 (segment (start 71.12 125.095) (end 70.485 125.73) (width 0.127) (layer F.Cu) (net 13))
 (segment (start 69.215 127) (end 70.485 125.73) (width 0.127) (layer B.Cu) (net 13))
 (segment (start 69.215 130.175) (end 69.215 127) (width 0.127) (layer B.Cu) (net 13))
 (segment (start 58.84 127.095) (end 69.12 127.095) (width 0.127) (layer B.Cu) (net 13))
 (via (at 63.005 125.73) (size 0.8) (drill 0.4) (layers F.Cu B.Cu) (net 14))
 (segment (start 58.84 125.825) (end 62.91 125.825) (width 0.127) (layer B.Cu) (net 14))
 (segment (start 62.91 125.825) (end 63.005 125.73) (width 0.127) (layer B.Cu) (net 14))
 (segment (start 67.31 128.905) (end 72.39 128.905) (width 0.127) (layer F.Cu) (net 14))
 (segment (start 72.39 128.905) (end 72.39 130.175) (width 0.127) (layer F.Cu) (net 14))
 (segment (start 63.5 128.905) (end 67.31 128.905) (width 0.127) (layer F.Cu) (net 14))
 (segment (start 63.005 125.73) (end 63.005 128.41) (width 0.127) (layer F.Cu) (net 14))
 (segment (start 63.005 128.41) (end 63.5 128.905) (width 0.127) (layer F.Cu) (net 14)))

